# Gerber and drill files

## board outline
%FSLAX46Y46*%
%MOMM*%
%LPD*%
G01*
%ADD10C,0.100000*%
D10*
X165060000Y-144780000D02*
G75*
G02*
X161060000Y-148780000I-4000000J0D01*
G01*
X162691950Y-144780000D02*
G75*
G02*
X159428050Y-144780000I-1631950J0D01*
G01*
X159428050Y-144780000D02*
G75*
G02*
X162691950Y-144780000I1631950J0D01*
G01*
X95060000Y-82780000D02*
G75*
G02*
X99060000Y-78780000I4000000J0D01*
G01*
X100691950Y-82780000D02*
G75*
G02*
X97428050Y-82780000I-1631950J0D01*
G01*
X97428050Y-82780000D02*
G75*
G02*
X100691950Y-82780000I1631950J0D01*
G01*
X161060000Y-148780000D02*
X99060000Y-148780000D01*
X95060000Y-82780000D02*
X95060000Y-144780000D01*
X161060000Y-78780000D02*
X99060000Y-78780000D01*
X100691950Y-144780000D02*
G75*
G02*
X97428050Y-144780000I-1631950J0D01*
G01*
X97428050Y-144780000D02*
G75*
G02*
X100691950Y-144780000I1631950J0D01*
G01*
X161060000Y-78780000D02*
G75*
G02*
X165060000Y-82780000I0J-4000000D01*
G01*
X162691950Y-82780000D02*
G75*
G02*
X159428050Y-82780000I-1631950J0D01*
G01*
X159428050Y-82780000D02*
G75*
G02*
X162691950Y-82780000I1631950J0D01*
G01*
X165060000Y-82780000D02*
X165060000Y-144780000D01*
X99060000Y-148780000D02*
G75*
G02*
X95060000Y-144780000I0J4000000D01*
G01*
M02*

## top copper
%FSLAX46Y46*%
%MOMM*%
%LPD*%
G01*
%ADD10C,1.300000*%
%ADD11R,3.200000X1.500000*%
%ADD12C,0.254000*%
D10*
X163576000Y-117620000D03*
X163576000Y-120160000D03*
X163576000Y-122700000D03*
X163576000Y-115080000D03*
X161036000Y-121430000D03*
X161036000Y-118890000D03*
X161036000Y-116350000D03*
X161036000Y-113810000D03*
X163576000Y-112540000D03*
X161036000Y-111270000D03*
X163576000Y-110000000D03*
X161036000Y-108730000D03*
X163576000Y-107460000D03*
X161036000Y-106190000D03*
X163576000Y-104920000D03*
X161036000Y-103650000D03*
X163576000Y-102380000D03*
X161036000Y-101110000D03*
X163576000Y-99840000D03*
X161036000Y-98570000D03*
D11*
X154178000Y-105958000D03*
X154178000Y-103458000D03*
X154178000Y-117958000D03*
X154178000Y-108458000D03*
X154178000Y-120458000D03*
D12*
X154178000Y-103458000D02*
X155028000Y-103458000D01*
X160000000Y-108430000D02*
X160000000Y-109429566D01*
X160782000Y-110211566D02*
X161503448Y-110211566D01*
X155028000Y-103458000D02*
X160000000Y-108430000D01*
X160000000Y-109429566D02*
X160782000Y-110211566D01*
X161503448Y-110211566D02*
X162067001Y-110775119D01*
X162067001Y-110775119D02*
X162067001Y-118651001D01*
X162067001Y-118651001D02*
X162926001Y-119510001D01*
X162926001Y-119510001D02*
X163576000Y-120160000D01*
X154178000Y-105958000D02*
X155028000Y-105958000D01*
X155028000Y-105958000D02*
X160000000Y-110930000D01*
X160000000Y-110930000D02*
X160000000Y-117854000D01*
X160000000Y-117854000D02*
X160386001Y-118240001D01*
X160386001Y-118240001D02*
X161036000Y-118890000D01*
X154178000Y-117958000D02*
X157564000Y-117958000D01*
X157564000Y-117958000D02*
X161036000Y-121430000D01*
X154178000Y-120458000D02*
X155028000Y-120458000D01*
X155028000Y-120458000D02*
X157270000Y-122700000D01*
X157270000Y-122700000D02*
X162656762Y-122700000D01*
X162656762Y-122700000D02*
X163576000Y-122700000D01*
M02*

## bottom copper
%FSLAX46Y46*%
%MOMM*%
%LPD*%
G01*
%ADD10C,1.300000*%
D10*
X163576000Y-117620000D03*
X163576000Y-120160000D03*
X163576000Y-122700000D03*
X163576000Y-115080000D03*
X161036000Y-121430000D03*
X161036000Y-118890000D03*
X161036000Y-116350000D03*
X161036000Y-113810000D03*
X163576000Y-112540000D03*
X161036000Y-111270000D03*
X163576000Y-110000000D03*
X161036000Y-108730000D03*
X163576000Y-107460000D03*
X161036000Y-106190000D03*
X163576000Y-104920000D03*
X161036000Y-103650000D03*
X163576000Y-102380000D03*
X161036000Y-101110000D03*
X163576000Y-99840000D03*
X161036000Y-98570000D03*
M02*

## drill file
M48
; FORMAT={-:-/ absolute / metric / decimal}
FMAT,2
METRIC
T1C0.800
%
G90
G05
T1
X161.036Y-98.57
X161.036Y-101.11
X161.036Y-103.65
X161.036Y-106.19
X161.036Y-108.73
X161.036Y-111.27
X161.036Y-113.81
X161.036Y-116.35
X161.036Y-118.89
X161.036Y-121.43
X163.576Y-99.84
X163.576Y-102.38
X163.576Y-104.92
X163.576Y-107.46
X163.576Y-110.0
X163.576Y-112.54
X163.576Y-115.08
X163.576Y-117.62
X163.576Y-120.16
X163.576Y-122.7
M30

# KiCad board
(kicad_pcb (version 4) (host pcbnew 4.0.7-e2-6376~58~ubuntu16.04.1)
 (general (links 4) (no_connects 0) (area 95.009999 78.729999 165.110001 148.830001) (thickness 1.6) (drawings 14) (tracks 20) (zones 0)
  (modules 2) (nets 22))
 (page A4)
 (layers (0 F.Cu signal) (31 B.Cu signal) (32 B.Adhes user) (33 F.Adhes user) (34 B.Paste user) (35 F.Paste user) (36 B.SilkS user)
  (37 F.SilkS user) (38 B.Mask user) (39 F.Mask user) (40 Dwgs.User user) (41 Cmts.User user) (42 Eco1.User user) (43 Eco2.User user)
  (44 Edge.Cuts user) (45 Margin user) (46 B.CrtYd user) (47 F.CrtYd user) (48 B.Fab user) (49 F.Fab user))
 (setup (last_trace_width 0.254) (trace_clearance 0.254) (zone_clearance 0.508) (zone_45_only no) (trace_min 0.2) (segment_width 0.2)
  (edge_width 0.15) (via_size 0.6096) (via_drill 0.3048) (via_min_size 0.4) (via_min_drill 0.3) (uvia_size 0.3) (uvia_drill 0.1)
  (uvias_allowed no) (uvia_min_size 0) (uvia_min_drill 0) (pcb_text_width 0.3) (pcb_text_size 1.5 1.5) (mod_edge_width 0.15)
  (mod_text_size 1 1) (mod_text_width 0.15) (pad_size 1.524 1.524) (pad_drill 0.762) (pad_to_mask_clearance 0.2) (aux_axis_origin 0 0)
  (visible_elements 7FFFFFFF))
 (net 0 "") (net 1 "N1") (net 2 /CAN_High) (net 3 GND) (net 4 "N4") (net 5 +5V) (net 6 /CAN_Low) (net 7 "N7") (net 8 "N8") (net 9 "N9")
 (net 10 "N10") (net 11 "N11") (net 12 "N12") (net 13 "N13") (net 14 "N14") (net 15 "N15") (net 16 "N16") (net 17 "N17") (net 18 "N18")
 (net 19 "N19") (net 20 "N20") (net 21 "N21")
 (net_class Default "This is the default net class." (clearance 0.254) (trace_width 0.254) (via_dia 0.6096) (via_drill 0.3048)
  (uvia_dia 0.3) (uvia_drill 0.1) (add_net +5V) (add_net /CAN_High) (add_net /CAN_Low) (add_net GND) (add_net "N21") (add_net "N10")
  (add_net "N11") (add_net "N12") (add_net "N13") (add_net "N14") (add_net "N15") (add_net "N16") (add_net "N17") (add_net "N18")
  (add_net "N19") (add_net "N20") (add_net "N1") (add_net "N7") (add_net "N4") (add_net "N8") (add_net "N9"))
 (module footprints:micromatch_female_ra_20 (layer F.Cu) (at 163.576 117.62 180)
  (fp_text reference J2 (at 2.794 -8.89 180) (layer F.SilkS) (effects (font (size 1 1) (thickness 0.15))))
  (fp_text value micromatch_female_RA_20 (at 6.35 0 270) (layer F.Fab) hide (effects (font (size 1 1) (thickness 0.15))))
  (pad 5 thru_hole circle (at 0 0 180) (size 1.3 1.3) (drill 0.8) (layers *.Cu *.Mask) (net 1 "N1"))
  (pad 3 thru_hole circle (at 0 -2.54 180) (size 1.3 1.3) (drill 0.8) (layers *.Cu *.Mask) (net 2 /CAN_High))
  (pad 1 thru_hole circle (at 0 -5.08 180) (size 1.3 1.3) (drill 0.8) (layers *.Cu *.Mask) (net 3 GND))
  (pad 7 thru_hole circle (at 0 2.54 180) (size 1.3 1.3) (drill 0.8) (layers *.Cu *.Mask) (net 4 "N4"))
  (pad 2 thru_hole circle (at 2.54 -3.81 180) (size 1.3 1.3) (drill 0.8) (layers *.Cu *.Mask) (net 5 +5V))
  (pad 4 thru_hole circle (at 2.54 -1.27 180) (size 1.3 1.3) (drill 0.8) (layers *.Cu *.Mask) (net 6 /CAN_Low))
  (pad 6 thru_hole circle (at 2.54 1.27 180) (size 1.3 1.3) (drill 0.8) (layers *.Cu *.Mask) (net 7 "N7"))
  (pad 8 thru_hole circle (at 2.54 3.81 180) (size 1.3 1.3) (drill 0.8) (layers *.Cu *.Mask) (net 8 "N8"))
  (pad 9 thru_hole circle (at 0 5.08 180) (size 1.3 1.3) (drill 0.8) (layers *.Cu *.Mask) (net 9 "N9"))
  (pad 10 thru_hole circle (at 2.54 6.35 180) (size 1.3 1.3) (drill 0.8) (layers *.Cu *.Mask) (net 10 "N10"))
  (pad 11 thru_hole circle (at 0 7.62 180) (size 1.3 1.3) (drill 0.8) (layers *.Cu *.Mask) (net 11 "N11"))
  (pad 12 thru_hole circle (at 2.54 8.89 180) (size 1.3 1.3) (drill 0.8) (layers *.Cu *.Mask) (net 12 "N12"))
  (pad 13 thru_hole circle (at 0 10.16 180) (size 1.3 1.3) (drill 0.8) (layers *.Cu *.Mask) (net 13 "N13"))
  (pad 14 thru_hole circle (at 2.54 11.43 180) (size 1.3 1.3) (drill 0.8) (layers *.Cu *.Mask) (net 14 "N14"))
  (pad 15 thru_hole circle (at 0 12.7 180) (size 1.3 1.3) (drill 0.8) (layers *.Cu *.Mask) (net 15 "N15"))
  (pad 16 thru_hole circle (at 2.54 13.97 180) (size 1.3 1.3) (drill 0.8) (layers *.Cu *.Mask) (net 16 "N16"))
  (pad 17 thru_hole circle (at 0 15.24 180) (size 1.3 1.3) (drill 0.8) (layers *.Cu *.Mask) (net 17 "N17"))
  (pad 18 thru_hole circle (at 2.54 16.51 180) (size 1.3 1.3) (drill 0.8) (layers *.Cu *.Mask) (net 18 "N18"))
  (pad 19 thru_hole circle (at 0 17.78 180) (size 1.3 1.3) (drill 0.8) (layers *.Cu *.Mask) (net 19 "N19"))
  (pad 20 thru_hole circle (at 2.54 19.05 180) (size 1.3 1.3) (drill 0.8) (layers *.Cu *.Mask) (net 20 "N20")))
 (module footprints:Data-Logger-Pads (layer F.Cu) (at 154.178 103.458 270)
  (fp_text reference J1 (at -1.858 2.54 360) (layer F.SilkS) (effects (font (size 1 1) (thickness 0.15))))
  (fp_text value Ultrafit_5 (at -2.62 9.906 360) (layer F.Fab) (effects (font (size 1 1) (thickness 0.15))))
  (pad 2 smd rect (at 2.5 0 270) (size 1.5 3.2) (layers F.Cu F.Paste F.Mask) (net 6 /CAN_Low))
  (pad 1 smd rect (at 0 0 270) (size 1.5 3.2) (layers F.Cu F.Paste F.Mask) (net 2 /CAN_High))
  (pad 4 smd rect (at 14.5 0 270) (size 1.5 3.2) (layers F.Cu F.Paste F.Mask) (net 5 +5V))
  (pad 3 smd rect (at 5 0 270) (size 1.5 3.2) (layers F.Cu F.Paste F.Mask) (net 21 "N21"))
  (pad 5 smd rect (at 17 0 270) (size 1.5 3.2) (layers F.Cu F.Paste F.Mask) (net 3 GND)))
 (gr_arc (start 161.06 144.78) (end 161.06 148.78) (angle -90) (layer Edge.Cuts) (width 0.1))
 (gr_circle (center 161.06 144.78) (end 162.69195 144.78) (layer Edge.Cuts) (width 0.1))
 (gr_arc (start 99.06 82.78) (end 99.06 78.78) (angle -90) (layer Edge.Cuts) (width 0.1))
 (gr_circle (center 99.06 82.78) (end 100.69195 82.78) (layer Edge.Cuts) (width 0.1))
 (gr_line (start 161.06 148.78) (end 99.06 148.78) (layer Edge.Cuts) (width 0.1))
 (gr_line (start 95.06 82.78) (end 95.06 144.78) (layer Edge.Cuts) (width 0.1))
 (gr_line (start 161.06 78.78) (end 99.06 78.78) (layer Edge.Cuts) (width 0.1))
 (gr_circle (center 99.06 144.78) (end 100.69195 144.78) (layer Edge.Cuts) (width 0.1))
 (gr_arc (start 161.06 82.78) (end 165.06 82.78) (angle -90) (layer Edge.Cuts) (width 0.1))
 (gr_circle (center 161.06 82.78) (end 162.69195 82.78) (layer Edge.Cuts) (width 0.1))
 (gr_line (start 165.06 82.78) (end 165.06 144.78) (layer Edge.Cuts) (width 0.1))
 (gr_arc (start 99.06 144.78) (end 95.06 144.78) (angle -90) (layer Edge.Cuts) (width 0.1))
 (segment (start 154.178 103.458) (end 155.028 103.458) (width 0.254) (layer F.Cu) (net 2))
 (segment (start 160 108.43) (end 160 109.429566) (width 0.254) (layer F.Cu) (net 2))
 (segment (start 160.782 110.211566) (end 161.503448 110.211566) (width 0.254) (layer F.Cu) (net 2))
 (segment (start 155.028 103.458) (end 160 108.43) (width 0.254) (layer F.Cu) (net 2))
 (segment (start 160 109.429566) (end 160.782 110.211566) (width 0.254) (layer F.Cu) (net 2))
 (segment (start 161.503448 110.211566) (end 162.067001 110.775119) (width 0.254) (layer F.Cu) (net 2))
 (segment (start 162.067001 110.775119) (end 162.067001 118.651001) (width 0.254) (layer F.Cu) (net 2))
 (segment (start 162.067001 118.651001) (end 162.926001 119.510001) (width 0.254) (layer F.Cu) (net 2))
 (segment (start 162.926001 119.510001) (end 163.576 120.16) (width 0.254) (layer F.Cu) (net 2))
 (segment (start 154.178 105.958) (end 155.028 105.958) (width 0.254) (layer F.Cu) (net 6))
 (segment (start 155.028 105.958) (end 160 110.93) (width 0.254) (layer F.Cu) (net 6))
 (segment (start 160 110.93) (end 160 117.854) (width 0.254) (layer F.Cu) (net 6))
 (segment (start 160 117.854) (end 160.386001 118.240001) (width 0.254) (layer F.Cu) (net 6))
 (segment (start 160.386001 118.240001) (end 161.036 118.89) (width 0.254) (layer F.Cu) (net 6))
 (segment (start 154.178 117.958) (end 157.564 117.958) (width 0.254) (layer F.Cu) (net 5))
 (segment (start 157.564 117.958) (end 161.036 121.43) (width 0.254) (layer F.Cu) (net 5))
 (segment (start 154.178 120.458) (end 155.028 120.458) (width 0.254) (layer F.Cu) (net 3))
 (segment (start 155.028 120.458) (end 157.27 122.7) (width 0.254) (layer F.Cu) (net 3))
 (segment (start 157.27 122.7) (end 162.656762 122.7) (width 0.254) (layer F.Cu) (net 3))
 (segment (start 162.656762 122.7) (end 163.576 122.7) (width 0.254) (layer F.Cu) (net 3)))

